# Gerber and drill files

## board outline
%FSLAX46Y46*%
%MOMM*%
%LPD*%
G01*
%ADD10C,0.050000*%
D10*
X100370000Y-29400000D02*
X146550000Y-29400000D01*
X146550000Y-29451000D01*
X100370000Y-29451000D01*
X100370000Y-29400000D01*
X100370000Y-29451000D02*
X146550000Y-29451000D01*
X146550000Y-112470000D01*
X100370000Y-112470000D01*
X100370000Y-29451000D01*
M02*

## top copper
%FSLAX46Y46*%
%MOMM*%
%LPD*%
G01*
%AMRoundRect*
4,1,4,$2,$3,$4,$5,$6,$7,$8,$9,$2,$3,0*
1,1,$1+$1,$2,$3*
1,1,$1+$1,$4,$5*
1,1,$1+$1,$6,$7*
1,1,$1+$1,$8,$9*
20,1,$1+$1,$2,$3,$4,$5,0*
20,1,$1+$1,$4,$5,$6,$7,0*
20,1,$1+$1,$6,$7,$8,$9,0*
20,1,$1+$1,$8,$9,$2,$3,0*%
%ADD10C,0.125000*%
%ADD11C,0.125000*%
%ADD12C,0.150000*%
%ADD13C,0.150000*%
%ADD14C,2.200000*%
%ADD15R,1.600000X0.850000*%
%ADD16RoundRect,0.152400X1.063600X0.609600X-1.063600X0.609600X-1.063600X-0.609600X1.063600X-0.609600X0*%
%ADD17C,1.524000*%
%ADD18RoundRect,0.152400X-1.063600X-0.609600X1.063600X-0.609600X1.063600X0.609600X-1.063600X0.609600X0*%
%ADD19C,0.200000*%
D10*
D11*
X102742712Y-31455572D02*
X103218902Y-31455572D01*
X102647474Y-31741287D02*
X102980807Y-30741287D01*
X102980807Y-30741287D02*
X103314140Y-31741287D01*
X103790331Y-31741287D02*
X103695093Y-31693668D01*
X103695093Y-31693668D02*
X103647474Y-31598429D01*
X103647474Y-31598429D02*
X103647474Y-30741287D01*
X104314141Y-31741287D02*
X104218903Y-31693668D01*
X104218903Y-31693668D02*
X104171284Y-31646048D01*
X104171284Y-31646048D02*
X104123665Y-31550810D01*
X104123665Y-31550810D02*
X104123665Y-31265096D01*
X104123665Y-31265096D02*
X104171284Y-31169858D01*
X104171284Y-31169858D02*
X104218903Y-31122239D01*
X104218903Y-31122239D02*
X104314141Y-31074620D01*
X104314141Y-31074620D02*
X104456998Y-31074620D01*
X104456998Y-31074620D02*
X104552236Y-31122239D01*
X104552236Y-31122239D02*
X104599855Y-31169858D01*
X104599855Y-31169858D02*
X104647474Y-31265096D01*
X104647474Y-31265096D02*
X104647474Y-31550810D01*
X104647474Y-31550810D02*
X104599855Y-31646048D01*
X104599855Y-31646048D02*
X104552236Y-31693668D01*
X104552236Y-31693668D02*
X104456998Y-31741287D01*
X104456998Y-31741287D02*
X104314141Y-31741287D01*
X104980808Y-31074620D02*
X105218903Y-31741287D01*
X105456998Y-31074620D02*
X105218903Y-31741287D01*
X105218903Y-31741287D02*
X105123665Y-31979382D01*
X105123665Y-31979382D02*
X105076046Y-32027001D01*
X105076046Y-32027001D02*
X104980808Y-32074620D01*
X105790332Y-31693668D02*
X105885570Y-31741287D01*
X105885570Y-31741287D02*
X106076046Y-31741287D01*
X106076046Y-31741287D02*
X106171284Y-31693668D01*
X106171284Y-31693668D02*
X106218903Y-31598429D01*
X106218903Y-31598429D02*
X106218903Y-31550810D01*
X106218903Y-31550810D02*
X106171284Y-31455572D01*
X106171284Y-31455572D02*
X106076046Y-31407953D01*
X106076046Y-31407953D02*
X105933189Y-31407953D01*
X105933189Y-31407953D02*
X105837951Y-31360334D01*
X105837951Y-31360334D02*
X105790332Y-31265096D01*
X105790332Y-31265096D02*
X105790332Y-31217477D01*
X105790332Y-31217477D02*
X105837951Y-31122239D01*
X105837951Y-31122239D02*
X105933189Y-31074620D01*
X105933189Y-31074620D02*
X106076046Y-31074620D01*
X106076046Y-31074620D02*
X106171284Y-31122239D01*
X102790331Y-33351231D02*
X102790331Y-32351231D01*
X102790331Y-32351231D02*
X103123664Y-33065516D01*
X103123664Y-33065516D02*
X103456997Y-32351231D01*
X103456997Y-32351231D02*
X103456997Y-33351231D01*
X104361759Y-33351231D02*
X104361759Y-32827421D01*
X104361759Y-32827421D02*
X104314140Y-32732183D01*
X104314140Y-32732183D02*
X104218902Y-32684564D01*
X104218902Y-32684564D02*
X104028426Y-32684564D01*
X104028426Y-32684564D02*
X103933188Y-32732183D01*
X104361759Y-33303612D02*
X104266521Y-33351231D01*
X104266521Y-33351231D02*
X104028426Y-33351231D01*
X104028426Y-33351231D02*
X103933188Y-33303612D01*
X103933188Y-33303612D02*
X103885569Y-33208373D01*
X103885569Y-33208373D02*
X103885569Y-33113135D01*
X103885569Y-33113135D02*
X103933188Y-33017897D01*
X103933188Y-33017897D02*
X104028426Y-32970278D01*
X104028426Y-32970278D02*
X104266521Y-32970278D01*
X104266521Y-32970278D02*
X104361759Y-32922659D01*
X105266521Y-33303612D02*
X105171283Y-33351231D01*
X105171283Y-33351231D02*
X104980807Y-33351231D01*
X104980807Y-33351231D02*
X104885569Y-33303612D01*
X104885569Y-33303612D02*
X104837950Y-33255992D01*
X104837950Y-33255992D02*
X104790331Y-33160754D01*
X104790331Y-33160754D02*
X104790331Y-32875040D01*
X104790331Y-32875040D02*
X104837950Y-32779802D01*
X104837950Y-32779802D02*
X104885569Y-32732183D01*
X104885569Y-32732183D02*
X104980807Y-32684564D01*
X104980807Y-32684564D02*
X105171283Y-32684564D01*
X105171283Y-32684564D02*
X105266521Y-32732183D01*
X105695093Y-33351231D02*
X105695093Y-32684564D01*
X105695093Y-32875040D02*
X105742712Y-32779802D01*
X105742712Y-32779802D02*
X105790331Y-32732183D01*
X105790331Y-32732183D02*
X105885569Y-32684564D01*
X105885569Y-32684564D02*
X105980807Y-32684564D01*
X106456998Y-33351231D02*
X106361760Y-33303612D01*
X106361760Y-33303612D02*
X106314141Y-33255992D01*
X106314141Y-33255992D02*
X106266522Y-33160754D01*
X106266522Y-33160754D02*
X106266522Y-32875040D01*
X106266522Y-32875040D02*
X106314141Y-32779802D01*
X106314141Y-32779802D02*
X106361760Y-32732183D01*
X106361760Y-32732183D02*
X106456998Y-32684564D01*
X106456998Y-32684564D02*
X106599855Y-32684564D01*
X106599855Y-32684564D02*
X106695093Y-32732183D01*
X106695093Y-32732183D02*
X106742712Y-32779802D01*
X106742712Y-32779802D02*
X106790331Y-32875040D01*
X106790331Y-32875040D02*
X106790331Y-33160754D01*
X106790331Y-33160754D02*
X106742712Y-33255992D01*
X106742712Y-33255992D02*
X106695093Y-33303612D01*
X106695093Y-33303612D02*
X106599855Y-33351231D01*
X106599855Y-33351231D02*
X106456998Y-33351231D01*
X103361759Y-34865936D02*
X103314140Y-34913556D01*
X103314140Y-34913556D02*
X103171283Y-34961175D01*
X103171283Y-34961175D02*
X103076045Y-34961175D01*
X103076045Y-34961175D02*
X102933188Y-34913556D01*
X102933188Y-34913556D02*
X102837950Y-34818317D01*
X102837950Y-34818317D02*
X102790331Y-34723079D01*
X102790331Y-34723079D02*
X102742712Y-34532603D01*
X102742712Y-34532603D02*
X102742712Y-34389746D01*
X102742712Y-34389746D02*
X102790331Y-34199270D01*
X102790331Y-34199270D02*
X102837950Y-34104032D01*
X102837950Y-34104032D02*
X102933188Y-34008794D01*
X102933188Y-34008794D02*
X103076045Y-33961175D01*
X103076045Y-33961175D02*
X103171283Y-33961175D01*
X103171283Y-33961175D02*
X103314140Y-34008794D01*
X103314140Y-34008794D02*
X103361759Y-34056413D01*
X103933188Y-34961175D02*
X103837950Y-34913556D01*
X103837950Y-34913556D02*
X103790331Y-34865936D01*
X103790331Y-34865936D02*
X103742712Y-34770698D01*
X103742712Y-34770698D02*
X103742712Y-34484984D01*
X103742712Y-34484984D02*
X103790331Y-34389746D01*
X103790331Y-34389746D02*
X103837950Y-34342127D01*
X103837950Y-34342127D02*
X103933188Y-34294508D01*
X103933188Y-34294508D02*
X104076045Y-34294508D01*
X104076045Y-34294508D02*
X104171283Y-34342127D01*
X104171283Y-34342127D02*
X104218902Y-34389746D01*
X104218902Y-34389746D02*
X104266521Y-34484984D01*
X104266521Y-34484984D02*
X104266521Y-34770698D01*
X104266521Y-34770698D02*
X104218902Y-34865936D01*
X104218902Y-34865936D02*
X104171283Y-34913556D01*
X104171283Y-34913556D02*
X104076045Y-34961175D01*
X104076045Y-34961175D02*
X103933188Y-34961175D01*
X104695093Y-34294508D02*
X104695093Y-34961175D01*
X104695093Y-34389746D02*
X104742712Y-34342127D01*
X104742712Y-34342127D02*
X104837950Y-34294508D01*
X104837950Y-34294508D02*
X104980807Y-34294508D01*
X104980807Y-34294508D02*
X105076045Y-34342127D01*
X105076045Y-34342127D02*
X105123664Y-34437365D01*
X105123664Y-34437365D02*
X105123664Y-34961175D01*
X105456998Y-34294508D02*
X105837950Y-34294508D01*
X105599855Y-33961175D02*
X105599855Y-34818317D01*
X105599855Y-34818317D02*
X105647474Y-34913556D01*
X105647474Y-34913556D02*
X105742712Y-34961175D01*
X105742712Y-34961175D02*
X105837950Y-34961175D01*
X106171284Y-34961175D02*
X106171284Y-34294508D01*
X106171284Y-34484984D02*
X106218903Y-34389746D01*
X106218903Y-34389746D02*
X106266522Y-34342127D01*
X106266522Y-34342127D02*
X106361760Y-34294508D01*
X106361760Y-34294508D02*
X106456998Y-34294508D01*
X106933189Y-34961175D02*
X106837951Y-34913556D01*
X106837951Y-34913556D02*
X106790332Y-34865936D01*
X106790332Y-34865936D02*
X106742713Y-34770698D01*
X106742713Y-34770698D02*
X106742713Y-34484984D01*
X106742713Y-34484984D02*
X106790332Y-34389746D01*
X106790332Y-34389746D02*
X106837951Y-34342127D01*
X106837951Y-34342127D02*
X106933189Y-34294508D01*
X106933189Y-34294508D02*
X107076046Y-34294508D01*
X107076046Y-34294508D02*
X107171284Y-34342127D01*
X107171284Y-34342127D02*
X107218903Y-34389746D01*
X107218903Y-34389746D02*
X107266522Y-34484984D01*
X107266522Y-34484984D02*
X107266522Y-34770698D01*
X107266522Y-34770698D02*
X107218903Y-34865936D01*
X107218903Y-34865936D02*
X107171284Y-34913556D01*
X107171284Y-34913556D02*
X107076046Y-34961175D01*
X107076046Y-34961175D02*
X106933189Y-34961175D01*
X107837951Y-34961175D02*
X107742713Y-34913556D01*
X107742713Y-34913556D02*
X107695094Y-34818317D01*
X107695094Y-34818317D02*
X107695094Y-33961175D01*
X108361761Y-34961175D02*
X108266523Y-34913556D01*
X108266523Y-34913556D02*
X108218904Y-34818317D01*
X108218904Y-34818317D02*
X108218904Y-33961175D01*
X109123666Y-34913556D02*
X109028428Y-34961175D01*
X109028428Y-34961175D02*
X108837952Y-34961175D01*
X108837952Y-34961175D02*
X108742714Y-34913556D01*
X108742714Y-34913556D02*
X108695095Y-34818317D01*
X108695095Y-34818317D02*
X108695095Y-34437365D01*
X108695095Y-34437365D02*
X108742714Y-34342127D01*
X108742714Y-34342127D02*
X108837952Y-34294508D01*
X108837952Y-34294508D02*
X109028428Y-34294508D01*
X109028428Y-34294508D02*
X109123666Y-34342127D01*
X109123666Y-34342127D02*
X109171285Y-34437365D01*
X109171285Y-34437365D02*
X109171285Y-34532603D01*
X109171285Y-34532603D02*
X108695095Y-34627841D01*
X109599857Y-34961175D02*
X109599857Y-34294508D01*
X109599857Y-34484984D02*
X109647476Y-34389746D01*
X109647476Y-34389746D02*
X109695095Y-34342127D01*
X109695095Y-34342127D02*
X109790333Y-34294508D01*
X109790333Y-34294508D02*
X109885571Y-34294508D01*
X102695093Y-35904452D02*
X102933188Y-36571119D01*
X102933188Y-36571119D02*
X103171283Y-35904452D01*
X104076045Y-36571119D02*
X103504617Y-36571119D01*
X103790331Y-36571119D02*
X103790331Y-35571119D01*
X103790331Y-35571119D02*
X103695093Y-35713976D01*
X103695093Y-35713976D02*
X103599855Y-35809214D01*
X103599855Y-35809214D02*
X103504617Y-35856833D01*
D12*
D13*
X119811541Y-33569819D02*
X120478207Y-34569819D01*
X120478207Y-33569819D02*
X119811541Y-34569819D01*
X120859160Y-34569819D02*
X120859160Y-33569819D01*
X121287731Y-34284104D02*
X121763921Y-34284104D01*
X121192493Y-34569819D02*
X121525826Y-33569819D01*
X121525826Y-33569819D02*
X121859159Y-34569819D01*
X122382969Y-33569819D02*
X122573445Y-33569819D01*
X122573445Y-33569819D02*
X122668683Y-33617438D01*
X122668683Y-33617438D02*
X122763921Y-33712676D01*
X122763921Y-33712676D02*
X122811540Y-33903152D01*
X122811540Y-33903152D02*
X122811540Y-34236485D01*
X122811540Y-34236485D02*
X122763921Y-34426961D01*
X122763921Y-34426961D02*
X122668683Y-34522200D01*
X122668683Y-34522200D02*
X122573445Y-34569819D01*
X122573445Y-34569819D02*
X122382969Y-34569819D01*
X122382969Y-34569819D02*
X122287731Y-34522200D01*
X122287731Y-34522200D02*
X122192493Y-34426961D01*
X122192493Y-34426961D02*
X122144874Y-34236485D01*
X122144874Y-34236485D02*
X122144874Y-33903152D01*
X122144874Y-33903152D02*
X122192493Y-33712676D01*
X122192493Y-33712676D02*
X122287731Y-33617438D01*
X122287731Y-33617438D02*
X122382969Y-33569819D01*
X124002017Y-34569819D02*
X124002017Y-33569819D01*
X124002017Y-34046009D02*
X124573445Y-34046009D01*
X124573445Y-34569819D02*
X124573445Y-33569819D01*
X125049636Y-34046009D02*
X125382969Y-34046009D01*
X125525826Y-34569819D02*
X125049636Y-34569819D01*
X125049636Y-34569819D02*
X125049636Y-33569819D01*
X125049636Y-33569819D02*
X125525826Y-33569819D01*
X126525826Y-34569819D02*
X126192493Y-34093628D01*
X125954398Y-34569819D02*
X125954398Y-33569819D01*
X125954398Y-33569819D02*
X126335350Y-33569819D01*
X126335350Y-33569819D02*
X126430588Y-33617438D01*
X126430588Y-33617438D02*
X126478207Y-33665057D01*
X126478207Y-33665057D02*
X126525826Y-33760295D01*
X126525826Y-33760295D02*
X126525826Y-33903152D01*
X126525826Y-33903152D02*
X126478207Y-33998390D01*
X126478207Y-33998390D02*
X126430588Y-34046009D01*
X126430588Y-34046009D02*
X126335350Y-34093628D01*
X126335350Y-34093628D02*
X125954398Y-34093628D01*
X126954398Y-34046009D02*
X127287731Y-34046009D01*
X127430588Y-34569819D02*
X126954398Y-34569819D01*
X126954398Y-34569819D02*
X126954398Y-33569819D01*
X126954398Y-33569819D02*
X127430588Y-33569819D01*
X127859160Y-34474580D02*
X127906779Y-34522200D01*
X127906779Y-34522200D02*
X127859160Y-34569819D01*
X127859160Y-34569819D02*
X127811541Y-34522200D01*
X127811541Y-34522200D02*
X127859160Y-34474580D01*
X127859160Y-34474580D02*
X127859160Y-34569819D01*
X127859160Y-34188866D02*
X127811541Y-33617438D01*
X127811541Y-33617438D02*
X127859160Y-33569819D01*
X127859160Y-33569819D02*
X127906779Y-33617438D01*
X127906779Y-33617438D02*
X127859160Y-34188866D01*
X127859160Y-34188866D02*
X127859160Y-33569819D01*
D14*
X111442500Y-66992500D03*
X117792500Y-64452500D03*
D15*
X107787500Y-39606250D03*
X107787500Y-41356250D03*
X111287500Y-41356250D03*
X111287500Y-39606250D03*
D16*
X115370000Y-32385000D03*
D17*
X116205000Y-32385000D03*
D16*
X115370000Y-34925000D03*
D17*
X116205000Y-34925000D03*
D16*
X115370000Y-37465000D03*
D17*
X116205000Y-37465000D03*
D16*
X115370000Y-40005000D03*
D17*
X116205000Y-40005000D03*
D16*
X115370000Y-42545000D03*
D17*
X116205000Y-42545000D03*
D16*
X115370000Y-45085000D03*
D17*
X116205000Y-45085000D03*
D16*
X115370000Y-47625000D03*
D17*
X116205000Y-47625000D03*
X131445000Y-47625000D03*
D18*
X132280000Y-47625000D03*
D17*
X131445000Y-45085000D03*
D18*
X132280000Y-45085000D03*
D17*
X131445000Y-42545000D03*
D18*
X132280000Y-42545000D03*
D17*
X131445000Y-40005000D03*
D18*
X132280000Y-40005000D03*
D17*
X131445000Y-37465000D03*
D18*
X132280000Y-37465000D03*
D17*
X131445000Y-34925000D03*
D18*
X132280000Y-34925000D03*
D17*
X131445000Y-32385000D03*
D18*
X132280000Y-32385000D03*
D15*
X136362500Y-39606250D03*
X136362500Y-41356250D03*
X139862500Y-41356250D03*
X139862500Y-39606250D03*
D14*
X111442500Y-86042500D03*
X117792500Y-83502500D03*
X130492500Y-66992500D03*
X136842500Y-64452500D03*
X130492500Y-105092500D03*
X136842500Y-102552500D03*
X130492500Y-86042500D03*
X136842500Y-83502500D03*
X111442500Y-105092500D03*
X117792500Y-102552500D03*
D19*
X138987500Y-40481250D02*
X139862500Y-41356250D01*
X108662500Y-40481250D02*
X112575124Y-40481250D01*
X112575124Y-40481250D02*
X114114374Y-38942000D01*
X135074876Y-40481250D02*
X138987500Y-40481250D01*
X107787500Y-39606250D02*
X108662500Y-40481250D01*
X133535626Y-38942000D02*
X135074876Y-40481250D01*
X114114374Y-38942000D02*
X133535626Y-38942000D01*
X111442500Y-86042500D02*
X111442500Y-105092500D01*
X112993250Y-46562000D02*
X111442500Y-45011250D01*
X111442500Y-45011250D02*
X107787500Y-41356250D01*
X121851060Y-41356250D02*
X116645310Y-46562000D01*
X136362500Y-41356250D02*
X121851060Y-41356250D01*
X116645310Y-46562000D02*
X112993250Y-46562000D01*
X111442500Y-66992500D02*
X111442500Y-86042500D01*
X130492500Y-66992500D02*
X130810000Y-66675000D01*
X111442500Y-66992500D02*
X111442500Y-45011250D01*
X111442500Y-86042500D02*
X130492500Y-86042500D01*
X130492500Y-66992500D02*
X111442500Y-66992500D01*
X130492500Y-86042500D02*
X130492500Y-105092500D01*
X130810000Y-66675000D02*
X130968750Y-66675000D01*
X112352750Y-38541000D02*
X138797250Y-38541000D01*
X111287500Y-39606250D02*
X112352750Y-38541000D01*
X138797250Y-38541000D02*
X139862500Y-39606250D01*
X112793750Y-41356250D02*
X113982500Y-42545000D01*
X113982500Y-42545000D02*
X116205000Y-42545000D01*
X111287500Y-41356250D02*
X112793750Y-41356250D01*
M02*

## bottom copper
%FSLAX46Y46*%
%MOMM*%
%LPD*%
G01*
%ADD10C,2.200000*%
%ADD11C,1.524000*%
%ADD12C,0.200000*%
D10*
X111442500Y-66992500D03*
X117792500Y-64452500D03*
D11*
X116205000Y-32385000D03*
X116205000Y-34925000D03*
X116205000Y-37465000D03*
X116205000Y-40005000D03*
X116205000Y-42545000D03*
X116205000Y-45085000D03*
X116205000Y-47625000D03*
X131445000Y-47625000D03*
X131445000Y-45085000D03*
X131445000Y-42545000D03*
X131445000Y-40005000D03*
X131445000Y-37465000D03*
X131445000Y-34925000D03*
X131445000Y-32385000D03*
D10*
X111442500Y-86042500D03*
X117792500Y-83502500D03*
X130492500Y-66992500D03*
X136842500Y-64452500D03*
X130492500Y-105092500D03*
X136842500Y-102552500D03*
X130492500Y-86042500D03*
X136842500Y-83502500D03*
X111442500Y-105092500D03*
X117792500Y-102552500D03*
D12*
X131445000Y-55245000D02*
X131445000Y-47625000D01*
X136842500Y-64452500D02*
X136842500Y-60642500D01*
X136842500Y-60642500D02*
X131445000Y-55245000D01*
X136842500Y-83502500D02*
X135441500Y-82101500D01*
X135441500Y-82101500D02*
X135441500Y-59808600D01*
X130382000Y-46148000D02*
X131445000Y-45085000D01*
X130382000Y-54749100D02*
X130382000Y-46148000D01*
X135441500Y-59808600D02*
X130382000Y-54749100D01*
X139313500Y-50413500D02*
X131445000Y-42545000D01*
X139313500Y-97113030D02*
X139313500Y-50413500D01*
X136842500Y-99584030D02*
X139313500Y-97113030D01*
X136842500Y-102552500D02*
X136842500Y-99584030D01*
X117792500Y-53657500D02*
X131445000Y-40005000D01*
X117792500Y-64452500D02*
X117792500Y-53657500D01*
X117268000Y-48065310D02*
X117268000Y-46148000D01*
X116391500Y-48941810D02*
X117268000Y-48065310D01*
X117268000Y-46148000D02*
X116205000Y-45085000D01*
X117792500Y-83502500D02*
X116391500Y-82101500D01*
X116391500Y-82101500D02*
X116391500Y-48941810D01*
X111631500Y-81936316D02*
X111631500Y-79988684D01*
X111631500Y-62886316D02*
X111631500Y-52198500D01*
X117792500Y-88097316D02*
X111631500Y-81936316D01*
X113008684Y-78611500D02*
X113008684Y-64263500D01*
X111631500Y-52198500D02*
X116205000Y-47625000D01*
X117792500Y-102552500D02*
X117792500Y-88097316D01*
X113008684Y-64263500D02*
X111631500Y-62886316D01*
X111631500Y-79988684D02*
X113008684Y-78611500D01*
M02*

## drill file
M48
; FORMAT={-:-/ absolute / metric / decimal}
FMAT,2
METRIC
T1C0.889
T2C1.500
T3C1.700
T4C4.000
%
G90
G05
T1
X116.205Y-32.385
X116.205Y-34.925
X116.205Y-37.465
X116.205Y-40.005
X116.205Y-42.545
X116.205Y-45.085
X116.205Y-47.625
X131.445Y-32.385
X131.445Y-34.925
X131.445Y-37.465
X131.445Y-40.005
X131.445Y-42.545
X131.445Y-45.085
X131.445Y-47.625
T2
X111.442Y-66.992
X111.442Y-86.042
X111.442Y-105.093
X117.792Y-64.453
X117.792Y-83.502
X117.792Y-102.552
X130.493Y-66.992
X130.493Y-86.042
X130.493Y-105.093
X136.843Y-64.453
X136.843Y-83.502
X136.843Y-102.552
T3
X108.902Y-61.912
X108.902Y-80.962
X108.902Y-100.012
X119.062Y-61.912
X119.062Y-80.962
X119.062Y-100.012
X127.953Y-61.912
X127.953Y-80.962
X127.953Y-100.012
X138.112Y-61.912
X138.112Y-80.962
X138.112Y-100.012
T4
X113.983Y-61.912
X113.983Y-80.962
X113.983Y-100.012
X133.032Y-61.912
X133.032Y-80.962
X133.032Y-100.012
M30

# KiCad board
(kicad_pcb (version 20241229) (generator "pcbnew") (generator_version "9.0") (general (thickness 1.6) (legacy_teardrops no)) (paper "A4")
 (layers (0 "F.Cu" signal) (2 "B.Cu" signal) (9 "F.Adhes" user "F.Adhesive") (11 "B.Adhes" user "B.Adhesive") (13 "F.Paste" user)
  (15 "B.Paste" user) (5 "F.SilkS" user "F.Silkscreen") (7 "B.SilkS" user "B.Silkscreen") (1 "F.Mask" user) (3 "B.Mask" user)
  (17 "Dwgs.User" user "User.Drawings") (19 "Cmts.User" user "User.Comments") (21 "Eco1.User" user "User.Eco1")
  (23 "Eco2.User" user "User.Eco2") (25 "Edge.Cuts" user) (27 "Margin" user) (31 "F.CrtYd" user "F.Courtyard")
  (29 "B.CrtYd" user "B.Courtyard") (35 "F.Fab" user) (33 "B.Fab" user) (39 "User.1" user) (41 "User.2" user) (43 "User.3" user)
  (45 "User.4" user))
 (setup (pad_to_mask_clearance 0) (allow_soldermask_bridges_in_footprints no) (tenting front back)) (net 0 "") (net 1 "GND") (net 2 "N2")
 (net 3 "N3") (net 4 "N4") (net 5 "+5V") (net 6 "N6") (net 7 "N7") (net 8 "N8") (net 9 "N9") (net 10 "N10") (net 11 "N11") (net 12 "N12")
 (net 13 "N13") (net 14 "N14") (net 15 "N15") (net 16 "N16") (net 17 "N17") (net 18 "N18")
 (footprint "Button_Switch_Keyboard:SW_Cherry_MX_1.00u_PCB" (layer "F.Cu") (at 111.4425 66.9925 180)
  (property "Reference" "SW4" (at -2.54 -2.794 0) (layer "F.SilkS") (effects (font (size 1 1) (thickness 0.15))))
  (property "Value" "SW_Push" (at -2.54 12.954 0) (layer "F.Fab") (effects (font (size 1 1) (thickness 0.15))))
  (pad "" np_thru_hole circle (at -7.62 5.08 180) (size 1.7 1.7) (drill 1.7) (layers "*.Cu" "*.Mask"))
  (pad "" np_thru_hole circle (at -2.54 5.08 180) (size 4 4) (drill 4) (layers "*.Cu" "*.Mask"))
  (pad "" np_thru_hole circle (at 2.54 5.08 180) (size 1.7 1.7) (drill 1.7) (layers "*.Cu" "*.Mask"))
  (pad "1" thru_hole circle (at 0 0 180) (size 2.2 2.2) (drill 1.5) (layers "*.Cu" "*.Mask") (remove_unused_layers no) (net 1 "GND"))
  (pad "2" thru_hole circle (at -6.35 2.54 180) (size 2.2 2.2) (drill 1.5) (layers "*.Cu" "*.Mask") (remove_unused_layers no) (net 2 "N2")))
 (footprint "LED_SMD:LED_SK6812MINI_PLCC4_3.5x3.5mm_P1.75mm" (layer "F.Cu") (at 109.5375 40.48125)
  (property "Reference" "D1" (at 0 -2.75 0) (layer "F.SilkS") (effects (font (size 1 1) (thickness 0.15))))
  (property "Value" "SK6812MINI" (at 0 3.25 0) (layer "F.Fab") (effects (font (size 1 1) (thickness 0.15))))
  (pad "1" smd rect (at -1.75 -0.875) (size 1.6 0.85) (layers "F.Cu" "F.Mask" "F.Paste") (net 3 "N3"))
  (pad "2" smd rect (at -1.75 0.875) (size 1.6 0.85) (layers "F.Cu" "F.Mask" "F.Paste") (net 1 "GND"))
  (pad "3" smd rect (at 1.75 0.875) (size 1.6 0.85) (layers "F.Cu" "F.Mask" "F.Paste") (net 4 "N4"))
  (pad "4" smd rect (at 1.75 -0.875) (size 1.6 0.85) (layers "F.Cu" "F.Mask" "F.Paste") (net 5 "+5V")))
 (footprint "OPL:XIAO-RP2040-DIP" (layer "F.Cu") (at 123.825 40.005)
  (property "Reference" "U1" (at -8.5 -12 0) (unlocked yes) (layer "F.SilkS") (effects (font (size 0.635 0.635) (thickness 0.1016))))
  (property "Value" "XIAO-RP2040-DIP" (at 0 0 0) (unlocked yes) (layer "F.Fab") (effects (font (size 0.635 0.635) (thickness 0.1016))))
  (pad "1" smd roundrect (at -8.455 -7.62 180) (size 2.432 1.524) (layers "F.Cu" "F.Mask") (roundrect_rratio 0.1) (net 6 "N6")
   (thermal_bridge_angle 45))
  (pad "1" thru_hole circle (at -7.62 -7.62 180) (size 1.524 1.524) (drill 0.889) (layers "*.Cu" "*.Mask") (remove_unused_layers no)
   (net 6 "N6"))
  (pad "2" smd roundrect (at -8.455 -5.08 180) (size 2.432 1.524) (layers "F.Cu" "F.Mask") (roundrect_rratio 0.1) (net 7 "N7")
   (thermal_bridge_angle 45))
  (pad "2" thru_hole circle (at -7.62 -5.08 180) (size 1.524 1.524) (drill 0.889) (layers "*.Cu" "*.Mask") (remove_unused_layers no)
   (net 7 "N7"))
  (pad "3" smd roundrect (at -8.455 -2.54 180) (size 2.432 1.524) (layers "F.Cu" "F.Mask") (roundrect_rratio 0.1) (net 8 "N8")
   (thermal_bridge_angle 45))
  (pad "3" thru_hole circle (at -7.62 -2.54 180) (size 1.524 1.524) (drill 0.889) (layers "*.Cu" "*.Mask") (remove_unused_layers no)
   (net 8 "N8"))
  (pad "4" smd roundrect (at -8.455 0 180) (size 2.432 1.524) (layers "F.Cu" "F.Mask") (roundrect_rratio 0.1) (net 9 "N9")
   (thermal_bridge_angle 45))
  (pad "4" thru_hole circle (at -7.62 0 180) (size 1.524 1.524) (drill 0.889) (layers "*.Cu" "*.Mask") (remove_unused_layers no)
   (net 9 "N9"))
  (pad "5" smd roundrect (at -8.455 2.54 180) (size 2.432 1.524) (layers "F.Cu" "F.Mask") (roundrect_rratio 0.1) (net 4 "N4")
   (thermal_bridge_angle 45))
  (pad "5" thru_hole circle (at -7.62 2.54 180) (size 1.524 1.524) (drill 0.889) (layers "*.Cu" "*.Mask") (remove_unused_layers no)
   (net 4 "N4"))
  (pad "6" smd roundrect (at -8.455 5.08 180) (size 2.432 1.524) (layers "F.Cu" "F.Mask") (roundrect_rratio 0.1) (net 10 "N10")
   (thermal_bridge_angle 45))
  (pad "6" thru_hole circle (at -7.62 5.08 180) (size 1.524 1.524) (drill 0.889) (layers "*.Cu" "*.Mask") (remove_unused_layers no)
   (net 10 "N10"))
  (pad "7" smd roundrect (at -8.455 7.62 180) (size 2.432 1.524) (layers "F.Cu" "F.Mask") (roundrect_rratio 0.1) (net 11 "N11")
   (thermal_bridge_angle 45))
  (pad "7" thru_hole circle (at -7.62 7.62 180) (size 1.524 1.524) (drill 0.889) (layers "*.Cu" "*.Mask") (remove_unused_layers no)
   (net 11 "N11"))
  (pad "8" thru_hole circle (at 7.62 7.62) (size 1.524 1.524) (drill 0.889) (layers "*.Cu" "*.Mask") (remove_unused_layers no)
   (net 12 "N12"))
  (pad "8" smd roundrect (at 8.455 7.62) (size 2.432 1.524) (layers "F.Cu" "F.Mask") (roundrect_rratio 0.1) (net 12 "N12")
   (thermal_bridge_angle 45))
  (pad "9" thru_hole circle (at 7.62 5.08) (size 1.524 1.524) (drill 0.889) (layers "*.Cu" "*.Mask") (remove_unused_layers no)
   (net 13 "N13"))
  (pad "9" smd roundrect (at 8.455 5.08) (size 2.432 1.524) (layers "F.Cu" "F.Mask") (roundrect_rratio 0.1) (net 13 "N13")
   (thermal_bridge_angle 45))
  (pad "10" thru_hole circle (at 7.62 2.54) (size 1.524 1.524) (drill 0.889) (layers "*.Cu" "*.Mask") (remove_unused_layers no)
   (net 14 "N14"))
  (pad "10" smd roundrect (at 8.455 2.54) (size 2.432 1.524) (layers "F.Cu" "F.Mask") (roundrect_rratio 0.1) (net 14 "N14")
   (thermal_bridge_angle 45))
  (pad "11" thru_hole circle (at 7.62 0) (size 1.524 1.524) (drill 0.889) (layers "*.Cu" "*.Mask") (remove_unused_layers no) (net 2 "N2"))
  (pad "11" smd roundrect (at 8.455 0) (size 2.432 1.524) (layers "F.Cu" "F.Mask") (roundrect_rratio 0.1) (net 2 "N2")
   (thermal_bridge_angle 45))
  (pad "12" thru_hole circle (at 7.62 -2.54) (size 1.524 1.524) (drill 0.889) (layers "*.Cu" "*.Mask") (remove_unused_layers no)
   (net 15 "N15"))
  (pad "12" smd roundrect (at 8.455 -2.54) (size 2.432 1.524) (layers "F.Cu" "F.Mask") (roundrect_rratio 0.1) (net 15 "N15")
   (thermal_bridge_angle 45))
  (pad "13" thru_hole circle (at 7.62 -5.08) (size 1.524 1.524) (drill 0.889) (layers "*.Cu" "*.Mask") (remove_unused_layers no)
   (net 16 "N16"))
  (pad "13" smd roundrect (at 8.455 -5.08) (size 2.432 1.524) (layers "F.Cu" "F.Mask") (roundrect_rratio 0.1) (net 16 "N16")
   (thermal_bridge_angle 45))
  (pad "14" thru_hole circle (at 7.62 -7.62) (size 1.524 1.524) (drill 0.889) (layers "*.Cu" "*.Mask") (remove_unused_layers no)
   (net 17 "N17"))
  (pad "14" smd roundrect (at 8.455 -7.62) (size 2.432 1.524) (layers "F.Cu" "F.Mask") (roundrect_rratio 0.1) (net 17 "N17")
   (thermal_bridge_angle 45)))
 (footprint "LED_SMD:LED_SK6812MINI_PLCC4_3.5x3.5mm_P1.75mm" (layer "F.Cu") (at 138.1125 40.48125)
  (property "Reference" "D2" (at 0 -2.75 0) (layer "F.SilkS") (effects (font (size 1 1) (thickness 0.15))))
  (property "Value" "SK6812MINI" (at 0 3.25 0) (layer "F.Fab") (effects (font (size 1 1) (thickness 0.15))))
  (pad "1" smd rect (at -1.75 -0.875) (size 1.6 0.85) (layers "F.Cu" "F.Mask" "F.Paste") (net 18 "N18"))
  (pad "2" smd rect (at -1.75 0.875) (size 1.6 0.85) (layers "F.Cu" "F.Mask" "F.Paste") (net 1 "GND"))
  (pad "3" smd rect (at 1.75 0.875) (size 1.6 0.85) (layers "F.Cu" "F.Mask" "F.Paste") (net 3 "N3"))
  (pad "4" smd rect (at 1.75 -0.875) (size 1.6 0.85) (layers "F.Cu" "F.Mask" "F.Paste") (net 5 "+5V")))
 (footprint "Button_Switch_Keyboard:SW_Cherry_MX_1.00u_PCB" (layer "F.Cu") (at 111.4425 86.0425 180)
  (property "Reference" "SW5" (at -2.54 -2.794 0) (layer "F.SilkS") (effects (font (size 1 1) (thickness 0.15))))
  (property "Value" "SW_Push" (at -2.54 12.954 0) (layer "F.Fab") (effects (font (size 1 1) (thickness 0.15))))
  (pad "" np_thru_hole circle (at -7.62 5.08 180) (size 1.7 1.7) (drill 1.7) (layers "*.Cu" "*.Mask"))
  (pad "" np_thru_hole circle (at -2.54 5.08 180) (size 4 4) (drill 4) (layers "*.Cu" "*.Mask"))
  (pad "" np_thru_hole circle (at 2.54 5.08 180) (size 1.7 1.7) (drill 1.7) (layers "*.Cu" "*.Mask"))
  (pad "1" thru_hole circle (at 0 0 180) (size 2.2 2.2) (drill 1.5) (layers "*.Cu" "*.Mask") (remove_unused_layers no) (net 1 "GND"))
  (pad "2" thru_hole circle (at -6.35 2.54 180) (size 2.2 2.2) (drill 1.5) (layers "*.Cu" "*.Mask") (remove_unused_layers no) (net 10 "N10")))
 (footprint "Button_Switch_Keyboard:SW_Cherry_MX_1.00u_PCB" (layer "F.Cu") (at 130.4925 66.9925 180)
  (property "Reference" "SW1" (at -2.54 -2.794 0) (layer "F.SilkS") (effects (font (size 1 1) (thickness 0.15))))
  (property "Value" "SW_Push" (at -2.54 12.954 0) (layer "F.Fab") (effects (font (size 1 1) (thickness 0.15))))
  (pad "" np_thru_hole circle (at -7.62 5.08 180) (size 1.7 1.7) (drill 1.7) (layers "*.Cu" "*.Mask"))
  (pad "" np_thru_hole circle (at -2.54 5.08 180) (size 4 4) (drill 4) (layers "*.Cu" "*.Mask"))
  (pad "" np_thru_hole circle (at 2.54 5.08 180) (size 1.7 1.7) (drill 1.7) (layers "*.Cu" "*.Mask"))
  (pad "1" thru_hole circle (at 0 0 180) (size 2.2 2.2) (drill 1.5) (layers "*.Cu" "*.Mask") (remove_unused_layers no) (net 1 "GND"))
  (pad "2" thru_hole circle (at -6.35 2.54 180) (size 2.2 2.2) (drill 1.5) (layers "*.Cu" "*.Mask") (remove_unused_layers no) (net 12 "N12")))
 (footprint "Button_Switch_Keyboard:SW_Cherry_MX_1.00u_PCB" (layer "F.Cu") (at 130.4925 105.0925 180)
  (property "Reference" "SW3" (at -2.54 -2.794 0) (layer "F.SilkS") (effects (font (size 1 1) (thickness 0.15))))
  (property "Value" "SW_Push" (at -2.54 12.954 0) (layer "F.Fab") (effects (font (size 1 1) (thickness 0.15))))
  (pad "" np_thru_hole circle (at -7.62 5.08 180) (size 1.7 1.7) (drill 1.7) (layers "*.Cu" "*.Mask"))
  (pad "" np_thru_hole circle (at -2.54 5.08 180) (size 4 4) (drill 4) (layers "*.Cu" "*.Mask"))
  (pad "" np_thru_hole circle (at 2.54 5.08 180) (size 1.7 1.7) (drill 1.7) (layers "*.Cu" "*.Mask"))
  (pad "1" thru_hole circle (at 0 0 180) (size 2.2 2.2) (drill 1.5) (layers "*.Cu" "*.Mask") (remove_unused_layers no) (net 1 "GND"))
  (pad "2" thru_hole circle (at -6.35 2.54 180) (size 2.2 2.2) (drill 1.5) (layers "*.Cu" "*.Mask") (remove_unused_layers no) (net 14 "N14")))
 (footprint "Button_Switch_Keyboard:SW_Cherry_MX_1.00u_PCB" (layer "F.Cu") (at 130.4925 86.0425 180)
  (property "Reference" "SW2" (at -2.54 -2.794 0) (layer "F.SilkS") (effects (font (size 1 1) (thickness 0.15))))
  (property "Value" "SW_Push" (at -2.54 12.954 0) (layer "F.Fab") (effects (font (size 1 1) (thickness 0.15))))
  (pad "" np_thru_hole circle (at -7.62 5.08 180) (size 1.7 1.7) (drill 1.7) (layers "*.Cu" "*.Mask"))
  (pad "" np_thru_hole circle (at -2.54 5.08 180) (size 4 4) (drill 4) (layers "*.Cu" "*.Mask"))
  (pad "" np_thru_hole circle (at 2.54 5.08 180) (size 1.7 1.7) (drill 1.7) (layers "*.Cu" "*.Mask"))
  (pad "1" thru_hole circle (at 0 0 180) (size 2.2 2.2) (drill 1.5) (layers "*.Cu" "*.Mask") (remove_unused_layers no) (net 1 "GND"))
  (pad "2" thru_hole circle (at -6.35 2.54 180) (size 2.2 2.2) (drill 1.5) (layers "*.Cu" "*.Mask") (remove_unused_layers no) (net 13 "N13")))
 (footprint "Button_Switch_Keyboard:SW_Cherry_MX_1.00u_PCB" (layer "F.Cu") (at 111.4425 105.0925 180)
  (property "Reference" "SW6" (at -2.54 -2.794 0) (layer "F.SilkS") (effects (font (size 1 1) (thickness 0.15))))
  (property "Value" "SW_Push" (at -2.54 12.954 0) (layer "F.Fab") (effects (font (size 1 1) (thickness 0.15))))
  (pad "" np_thru_hole circle (at -7.62 5.08 180) (size 1.7 1.7) (drill 1.7) (layers "*.Cu" "*.Mask"))
  (pad "" np_thru_hole circle (at -2.54 5.08 180) (size 4 4) (drill 4) (layers "*.Cu" "*.Mask"))
  (pad "" np_thru_hole circle (at 2.54 5.08 180) (size 1.7 1.7) (drill 1.7) (layers "*.Cu" "*.Mask"))
  (pad "1" thru_hole circle (at 0 0 180) (size 2.2 2.2) (drill 1.5) (layers "*.Cu" "*.Mask") (remove_unused_layers no) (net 1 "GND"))
  (pad "2" thru_hole circle (at -6.35 2.54 180) (size 2.2 2.2) (drill 1.5) (layers "*.Cu" "*.Mask") (remove_unused_layers no) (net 11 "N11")))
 (gr_rect (start 100.37 29.4) (end 146.55 29.451) (stroke (width 0.05) (type default)) (fill no) (layer "Edge.Cuts"))
 (gr_rect (start 100.37 29.451) (end 146.55 112.47) (stroke (width 0.05) (type default)) (fill no) (layer "Edge.Cuts"))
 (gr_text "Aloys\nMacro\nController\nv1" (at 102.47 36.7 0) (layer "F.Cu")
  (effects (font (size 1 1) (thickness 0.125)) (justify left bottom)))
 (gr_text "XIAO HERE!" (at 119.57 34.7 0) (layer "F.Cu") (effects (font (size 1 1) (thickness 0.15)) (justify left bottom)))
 (segment (start 138.9875 40.48125) (end 139.8625 41.35625) (width 0.2) (layer "F.Cu") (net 3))
 (segment (start 108.6625 40.48125) (end 112.575124 40.48125) (width 0.2) (layer "F.Cu") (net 3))
 (segment (start 112.575124 40.48125) (end 114.114374 38.942) (width 0.2) (layer "F.Cu") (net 3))
 (segment (start 135.074876 40.48125) (end 138.9875 40.48125) (width 0.2) (layer "F.Cu") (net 3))
 (segment (start 107.7875 39.60625) (end 108.6625 40.48125) (width 0.2) (layer "F.Cu") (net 3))
 (segment (start 133.535626 38.942) (end 135.074876 40.48125) (width 0.2) (layer "F.Cu") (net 3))
 (segment (start 114.114374 38.942) (end 133.535626 38.942) (width 0.2) (layer "F.Cu") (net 3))
 (segment (start 111.4425 86.0425) (end 111.4425 105.0925) (width 0.2) (layer "F.Cu") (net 1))
 (segment (start 112.99325 46.562) (end 111.4425 45.01125) (width 0.2) (layer "F.Cu") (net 1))
 (segment (start 111.4425 45.01125) (end 107.7875 41.35625) (width 0.2) (layer "F.Cu") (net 1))
 (segment (start 121.85106 41.35625) (end 116.64531 46.562) (width 0.2) (layer "F.Cu") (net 1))
 (segment (start 136.3625 41.35625) (end 121.85106 41.35625) (width 0.2) (layer "F.Cu") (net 1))
 (segment (start 116.64531 46.562) (end 112.99325 46.562) (width 0.2) (layer "F.Cu") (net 1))
 (segment (start 111.4425 66.9925) (end 111.4425 86.0425) (width 0.2) (layer "F.Cu") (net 1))
 (segment (start 130.4925 66.9925) (end 130.81 66.675) (width 0.2) (layer "F.Cu") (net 1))
 (segment (start 111.4425 66.9925) (end 111.4425 45.01125) (width 0.2) (layer "F.Cu") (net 1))
 (segment (start 111.4425 86.0425) (end 130.4925 86.0425) (width 0.2) (layer "F.Cu") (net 1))
 (segment (start 130.4925 66.9925) (end 111.4425 66.9925) (width 0.2) (layer "F.Cu") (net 1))
 (segment (start 130.4925 86.0425) (end 130.4925 105.0925) (width 0.2) (layer "F.Cu") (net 1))
 (segment (start 130.81 66.675) (end 130.96875 66.675) (width 0.2) (layer "F.Cu") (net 1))
 (segment (start 112.35275 38.541) (end 138.79725 38.541) (width 0.2) (layer "F.Cu") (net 5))
 (segment (start 111.2875 39.60625) (end 112.35275 38.541) (width 0.2) (layer "F.Cu") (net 5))
 (segment (start 138.79725 38.541) (end 139.8625 39.60625) (width 0.2) (layer "F.Cu") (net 5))
 (segment (start 112.79375 41.35625) (end 113.9825 42.545) (width 0.2) (layer "F.Cu") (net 4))
 (segment (start 113.9825 42.545) (end 116.205 42.545) (width 0.2) (layer "F.Cu") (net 4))
 (segment (start 111.2875 41.35625) (end 112.79375 41.35625) (width 0.2) (layer "F.Cu") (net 4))
 (segment (start 131.445 55.245) (end 131.445 47.625) (width 0.2) (layer "B.Cu") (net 12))
 (segment (start 136.8425 64.4525) (end 136.8425 60.6425) (width 0.2) (layer "B.Cu") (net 12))
 (segment (start 136.8425 60.6425) (end 131.445 55.245) (width 0.2) (layer "B.Cu") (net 12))
 (segment (start 136.8425 83.5025) (end 135.4415 82.1015) (width 0.2) (layer "B.Cu") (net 13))
 (segment (start 135.4415 82.1015) (end 135.4415 59.8086) (width 0.2) (layer "B.Cu") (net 13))
 (segment (start 130.382 46.148) (end 131.445 45.085) (width 0.2) (layer "B.Cu") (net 13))
 (segment (start 130.382 54.7491) (end 130.382 46.148) (width 0.2) (layer "B.Cu") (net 13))
 (segment (start 135.4415 59.8086) (end 130.382 54.7491) (width 0.2) (layer "B.Cu") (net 13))
 (segment (start 139.3135 50.4135) (end 131.445 42.545) (width 0.2) (layer "B.Cu") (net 14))
 (segment (start 139.3135 97.11303) (end 139.3135 50.4135) (width 0.2) (layer "B.Cu") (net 14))
 (segment (start 136.8425 99.58403) (end 139.3135 97.11303) (width 0.2) (layer "B.Cu") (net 14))
 (segment (start 136.8425 102.5525) (end 136.8425 99.58403) (width 0.2) (layer "B.Cu") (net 14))
 (segment (start 117.7925 53.6575) (end 131.445 40.005) (width 0.2) (layer "B.Cu") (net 2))
 (segment (start 117.7925 64.4525) (end 117.7925 53.6575) (width 0.2) (layer "B.Cu") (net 2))
 (segment (start 117.268 48.06531) (end 117.268 46.148) (width 0.2) (layer "B.Cu") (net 10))
 (segment (start 116.3915 48.94181) (end 117.268 48.06531) (width 0.2) (layer "B.Cu") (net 10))
 (segment (start 117.268 46.148) (end 116.205 45.085) (width 0.2) (layer "B.Cu") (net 10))
 (segment (start 117.7925 83.5025) (end 116.3915 82.1015) (width 0.2) (layer "B.Cu") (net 10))
 (segment (start 116.3915 82.1015) (end 116.3915 48.94181) (width 0.2) (layer "B.Cu") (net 10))
 (segment (start 111.6315 81.936316) (end 111.6315 79.988684) (width 0.2) (layer "B.Cu") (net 11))
 (segment (start 111.6315 62.886316) (end 111.6315 52.1985) (width 0.2) (layer "B.Cu") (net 11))
 (segment (start 117.7925 88.097316) (end 111.6315 81.936316) (width 0.2) (layer "B.Cu") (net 11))
 (segment (start 113.008684 78.6115) (end 113.008684 64.2635) (width 0.2) (layer "B.Cu") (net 11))
 (segment (start 111.6315 52.1985) (end 116.205 47.625) (width 0.2) (layer "B.Cu") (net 11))
 (segment (start 117.7925 102.5525) (end 117.7925 88.097316) (width 0.2) (layer "B.Cu") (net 11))
 (segment (start 113.008684 64.2635) (end 111.6315 62.886316) (width 0.2) (layer "B.Cu") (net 11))
 (segment (start 111.6315 79.988684) (end 113.008684 78.6115) (width 0.2) (layer "B.Cu") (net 11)))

